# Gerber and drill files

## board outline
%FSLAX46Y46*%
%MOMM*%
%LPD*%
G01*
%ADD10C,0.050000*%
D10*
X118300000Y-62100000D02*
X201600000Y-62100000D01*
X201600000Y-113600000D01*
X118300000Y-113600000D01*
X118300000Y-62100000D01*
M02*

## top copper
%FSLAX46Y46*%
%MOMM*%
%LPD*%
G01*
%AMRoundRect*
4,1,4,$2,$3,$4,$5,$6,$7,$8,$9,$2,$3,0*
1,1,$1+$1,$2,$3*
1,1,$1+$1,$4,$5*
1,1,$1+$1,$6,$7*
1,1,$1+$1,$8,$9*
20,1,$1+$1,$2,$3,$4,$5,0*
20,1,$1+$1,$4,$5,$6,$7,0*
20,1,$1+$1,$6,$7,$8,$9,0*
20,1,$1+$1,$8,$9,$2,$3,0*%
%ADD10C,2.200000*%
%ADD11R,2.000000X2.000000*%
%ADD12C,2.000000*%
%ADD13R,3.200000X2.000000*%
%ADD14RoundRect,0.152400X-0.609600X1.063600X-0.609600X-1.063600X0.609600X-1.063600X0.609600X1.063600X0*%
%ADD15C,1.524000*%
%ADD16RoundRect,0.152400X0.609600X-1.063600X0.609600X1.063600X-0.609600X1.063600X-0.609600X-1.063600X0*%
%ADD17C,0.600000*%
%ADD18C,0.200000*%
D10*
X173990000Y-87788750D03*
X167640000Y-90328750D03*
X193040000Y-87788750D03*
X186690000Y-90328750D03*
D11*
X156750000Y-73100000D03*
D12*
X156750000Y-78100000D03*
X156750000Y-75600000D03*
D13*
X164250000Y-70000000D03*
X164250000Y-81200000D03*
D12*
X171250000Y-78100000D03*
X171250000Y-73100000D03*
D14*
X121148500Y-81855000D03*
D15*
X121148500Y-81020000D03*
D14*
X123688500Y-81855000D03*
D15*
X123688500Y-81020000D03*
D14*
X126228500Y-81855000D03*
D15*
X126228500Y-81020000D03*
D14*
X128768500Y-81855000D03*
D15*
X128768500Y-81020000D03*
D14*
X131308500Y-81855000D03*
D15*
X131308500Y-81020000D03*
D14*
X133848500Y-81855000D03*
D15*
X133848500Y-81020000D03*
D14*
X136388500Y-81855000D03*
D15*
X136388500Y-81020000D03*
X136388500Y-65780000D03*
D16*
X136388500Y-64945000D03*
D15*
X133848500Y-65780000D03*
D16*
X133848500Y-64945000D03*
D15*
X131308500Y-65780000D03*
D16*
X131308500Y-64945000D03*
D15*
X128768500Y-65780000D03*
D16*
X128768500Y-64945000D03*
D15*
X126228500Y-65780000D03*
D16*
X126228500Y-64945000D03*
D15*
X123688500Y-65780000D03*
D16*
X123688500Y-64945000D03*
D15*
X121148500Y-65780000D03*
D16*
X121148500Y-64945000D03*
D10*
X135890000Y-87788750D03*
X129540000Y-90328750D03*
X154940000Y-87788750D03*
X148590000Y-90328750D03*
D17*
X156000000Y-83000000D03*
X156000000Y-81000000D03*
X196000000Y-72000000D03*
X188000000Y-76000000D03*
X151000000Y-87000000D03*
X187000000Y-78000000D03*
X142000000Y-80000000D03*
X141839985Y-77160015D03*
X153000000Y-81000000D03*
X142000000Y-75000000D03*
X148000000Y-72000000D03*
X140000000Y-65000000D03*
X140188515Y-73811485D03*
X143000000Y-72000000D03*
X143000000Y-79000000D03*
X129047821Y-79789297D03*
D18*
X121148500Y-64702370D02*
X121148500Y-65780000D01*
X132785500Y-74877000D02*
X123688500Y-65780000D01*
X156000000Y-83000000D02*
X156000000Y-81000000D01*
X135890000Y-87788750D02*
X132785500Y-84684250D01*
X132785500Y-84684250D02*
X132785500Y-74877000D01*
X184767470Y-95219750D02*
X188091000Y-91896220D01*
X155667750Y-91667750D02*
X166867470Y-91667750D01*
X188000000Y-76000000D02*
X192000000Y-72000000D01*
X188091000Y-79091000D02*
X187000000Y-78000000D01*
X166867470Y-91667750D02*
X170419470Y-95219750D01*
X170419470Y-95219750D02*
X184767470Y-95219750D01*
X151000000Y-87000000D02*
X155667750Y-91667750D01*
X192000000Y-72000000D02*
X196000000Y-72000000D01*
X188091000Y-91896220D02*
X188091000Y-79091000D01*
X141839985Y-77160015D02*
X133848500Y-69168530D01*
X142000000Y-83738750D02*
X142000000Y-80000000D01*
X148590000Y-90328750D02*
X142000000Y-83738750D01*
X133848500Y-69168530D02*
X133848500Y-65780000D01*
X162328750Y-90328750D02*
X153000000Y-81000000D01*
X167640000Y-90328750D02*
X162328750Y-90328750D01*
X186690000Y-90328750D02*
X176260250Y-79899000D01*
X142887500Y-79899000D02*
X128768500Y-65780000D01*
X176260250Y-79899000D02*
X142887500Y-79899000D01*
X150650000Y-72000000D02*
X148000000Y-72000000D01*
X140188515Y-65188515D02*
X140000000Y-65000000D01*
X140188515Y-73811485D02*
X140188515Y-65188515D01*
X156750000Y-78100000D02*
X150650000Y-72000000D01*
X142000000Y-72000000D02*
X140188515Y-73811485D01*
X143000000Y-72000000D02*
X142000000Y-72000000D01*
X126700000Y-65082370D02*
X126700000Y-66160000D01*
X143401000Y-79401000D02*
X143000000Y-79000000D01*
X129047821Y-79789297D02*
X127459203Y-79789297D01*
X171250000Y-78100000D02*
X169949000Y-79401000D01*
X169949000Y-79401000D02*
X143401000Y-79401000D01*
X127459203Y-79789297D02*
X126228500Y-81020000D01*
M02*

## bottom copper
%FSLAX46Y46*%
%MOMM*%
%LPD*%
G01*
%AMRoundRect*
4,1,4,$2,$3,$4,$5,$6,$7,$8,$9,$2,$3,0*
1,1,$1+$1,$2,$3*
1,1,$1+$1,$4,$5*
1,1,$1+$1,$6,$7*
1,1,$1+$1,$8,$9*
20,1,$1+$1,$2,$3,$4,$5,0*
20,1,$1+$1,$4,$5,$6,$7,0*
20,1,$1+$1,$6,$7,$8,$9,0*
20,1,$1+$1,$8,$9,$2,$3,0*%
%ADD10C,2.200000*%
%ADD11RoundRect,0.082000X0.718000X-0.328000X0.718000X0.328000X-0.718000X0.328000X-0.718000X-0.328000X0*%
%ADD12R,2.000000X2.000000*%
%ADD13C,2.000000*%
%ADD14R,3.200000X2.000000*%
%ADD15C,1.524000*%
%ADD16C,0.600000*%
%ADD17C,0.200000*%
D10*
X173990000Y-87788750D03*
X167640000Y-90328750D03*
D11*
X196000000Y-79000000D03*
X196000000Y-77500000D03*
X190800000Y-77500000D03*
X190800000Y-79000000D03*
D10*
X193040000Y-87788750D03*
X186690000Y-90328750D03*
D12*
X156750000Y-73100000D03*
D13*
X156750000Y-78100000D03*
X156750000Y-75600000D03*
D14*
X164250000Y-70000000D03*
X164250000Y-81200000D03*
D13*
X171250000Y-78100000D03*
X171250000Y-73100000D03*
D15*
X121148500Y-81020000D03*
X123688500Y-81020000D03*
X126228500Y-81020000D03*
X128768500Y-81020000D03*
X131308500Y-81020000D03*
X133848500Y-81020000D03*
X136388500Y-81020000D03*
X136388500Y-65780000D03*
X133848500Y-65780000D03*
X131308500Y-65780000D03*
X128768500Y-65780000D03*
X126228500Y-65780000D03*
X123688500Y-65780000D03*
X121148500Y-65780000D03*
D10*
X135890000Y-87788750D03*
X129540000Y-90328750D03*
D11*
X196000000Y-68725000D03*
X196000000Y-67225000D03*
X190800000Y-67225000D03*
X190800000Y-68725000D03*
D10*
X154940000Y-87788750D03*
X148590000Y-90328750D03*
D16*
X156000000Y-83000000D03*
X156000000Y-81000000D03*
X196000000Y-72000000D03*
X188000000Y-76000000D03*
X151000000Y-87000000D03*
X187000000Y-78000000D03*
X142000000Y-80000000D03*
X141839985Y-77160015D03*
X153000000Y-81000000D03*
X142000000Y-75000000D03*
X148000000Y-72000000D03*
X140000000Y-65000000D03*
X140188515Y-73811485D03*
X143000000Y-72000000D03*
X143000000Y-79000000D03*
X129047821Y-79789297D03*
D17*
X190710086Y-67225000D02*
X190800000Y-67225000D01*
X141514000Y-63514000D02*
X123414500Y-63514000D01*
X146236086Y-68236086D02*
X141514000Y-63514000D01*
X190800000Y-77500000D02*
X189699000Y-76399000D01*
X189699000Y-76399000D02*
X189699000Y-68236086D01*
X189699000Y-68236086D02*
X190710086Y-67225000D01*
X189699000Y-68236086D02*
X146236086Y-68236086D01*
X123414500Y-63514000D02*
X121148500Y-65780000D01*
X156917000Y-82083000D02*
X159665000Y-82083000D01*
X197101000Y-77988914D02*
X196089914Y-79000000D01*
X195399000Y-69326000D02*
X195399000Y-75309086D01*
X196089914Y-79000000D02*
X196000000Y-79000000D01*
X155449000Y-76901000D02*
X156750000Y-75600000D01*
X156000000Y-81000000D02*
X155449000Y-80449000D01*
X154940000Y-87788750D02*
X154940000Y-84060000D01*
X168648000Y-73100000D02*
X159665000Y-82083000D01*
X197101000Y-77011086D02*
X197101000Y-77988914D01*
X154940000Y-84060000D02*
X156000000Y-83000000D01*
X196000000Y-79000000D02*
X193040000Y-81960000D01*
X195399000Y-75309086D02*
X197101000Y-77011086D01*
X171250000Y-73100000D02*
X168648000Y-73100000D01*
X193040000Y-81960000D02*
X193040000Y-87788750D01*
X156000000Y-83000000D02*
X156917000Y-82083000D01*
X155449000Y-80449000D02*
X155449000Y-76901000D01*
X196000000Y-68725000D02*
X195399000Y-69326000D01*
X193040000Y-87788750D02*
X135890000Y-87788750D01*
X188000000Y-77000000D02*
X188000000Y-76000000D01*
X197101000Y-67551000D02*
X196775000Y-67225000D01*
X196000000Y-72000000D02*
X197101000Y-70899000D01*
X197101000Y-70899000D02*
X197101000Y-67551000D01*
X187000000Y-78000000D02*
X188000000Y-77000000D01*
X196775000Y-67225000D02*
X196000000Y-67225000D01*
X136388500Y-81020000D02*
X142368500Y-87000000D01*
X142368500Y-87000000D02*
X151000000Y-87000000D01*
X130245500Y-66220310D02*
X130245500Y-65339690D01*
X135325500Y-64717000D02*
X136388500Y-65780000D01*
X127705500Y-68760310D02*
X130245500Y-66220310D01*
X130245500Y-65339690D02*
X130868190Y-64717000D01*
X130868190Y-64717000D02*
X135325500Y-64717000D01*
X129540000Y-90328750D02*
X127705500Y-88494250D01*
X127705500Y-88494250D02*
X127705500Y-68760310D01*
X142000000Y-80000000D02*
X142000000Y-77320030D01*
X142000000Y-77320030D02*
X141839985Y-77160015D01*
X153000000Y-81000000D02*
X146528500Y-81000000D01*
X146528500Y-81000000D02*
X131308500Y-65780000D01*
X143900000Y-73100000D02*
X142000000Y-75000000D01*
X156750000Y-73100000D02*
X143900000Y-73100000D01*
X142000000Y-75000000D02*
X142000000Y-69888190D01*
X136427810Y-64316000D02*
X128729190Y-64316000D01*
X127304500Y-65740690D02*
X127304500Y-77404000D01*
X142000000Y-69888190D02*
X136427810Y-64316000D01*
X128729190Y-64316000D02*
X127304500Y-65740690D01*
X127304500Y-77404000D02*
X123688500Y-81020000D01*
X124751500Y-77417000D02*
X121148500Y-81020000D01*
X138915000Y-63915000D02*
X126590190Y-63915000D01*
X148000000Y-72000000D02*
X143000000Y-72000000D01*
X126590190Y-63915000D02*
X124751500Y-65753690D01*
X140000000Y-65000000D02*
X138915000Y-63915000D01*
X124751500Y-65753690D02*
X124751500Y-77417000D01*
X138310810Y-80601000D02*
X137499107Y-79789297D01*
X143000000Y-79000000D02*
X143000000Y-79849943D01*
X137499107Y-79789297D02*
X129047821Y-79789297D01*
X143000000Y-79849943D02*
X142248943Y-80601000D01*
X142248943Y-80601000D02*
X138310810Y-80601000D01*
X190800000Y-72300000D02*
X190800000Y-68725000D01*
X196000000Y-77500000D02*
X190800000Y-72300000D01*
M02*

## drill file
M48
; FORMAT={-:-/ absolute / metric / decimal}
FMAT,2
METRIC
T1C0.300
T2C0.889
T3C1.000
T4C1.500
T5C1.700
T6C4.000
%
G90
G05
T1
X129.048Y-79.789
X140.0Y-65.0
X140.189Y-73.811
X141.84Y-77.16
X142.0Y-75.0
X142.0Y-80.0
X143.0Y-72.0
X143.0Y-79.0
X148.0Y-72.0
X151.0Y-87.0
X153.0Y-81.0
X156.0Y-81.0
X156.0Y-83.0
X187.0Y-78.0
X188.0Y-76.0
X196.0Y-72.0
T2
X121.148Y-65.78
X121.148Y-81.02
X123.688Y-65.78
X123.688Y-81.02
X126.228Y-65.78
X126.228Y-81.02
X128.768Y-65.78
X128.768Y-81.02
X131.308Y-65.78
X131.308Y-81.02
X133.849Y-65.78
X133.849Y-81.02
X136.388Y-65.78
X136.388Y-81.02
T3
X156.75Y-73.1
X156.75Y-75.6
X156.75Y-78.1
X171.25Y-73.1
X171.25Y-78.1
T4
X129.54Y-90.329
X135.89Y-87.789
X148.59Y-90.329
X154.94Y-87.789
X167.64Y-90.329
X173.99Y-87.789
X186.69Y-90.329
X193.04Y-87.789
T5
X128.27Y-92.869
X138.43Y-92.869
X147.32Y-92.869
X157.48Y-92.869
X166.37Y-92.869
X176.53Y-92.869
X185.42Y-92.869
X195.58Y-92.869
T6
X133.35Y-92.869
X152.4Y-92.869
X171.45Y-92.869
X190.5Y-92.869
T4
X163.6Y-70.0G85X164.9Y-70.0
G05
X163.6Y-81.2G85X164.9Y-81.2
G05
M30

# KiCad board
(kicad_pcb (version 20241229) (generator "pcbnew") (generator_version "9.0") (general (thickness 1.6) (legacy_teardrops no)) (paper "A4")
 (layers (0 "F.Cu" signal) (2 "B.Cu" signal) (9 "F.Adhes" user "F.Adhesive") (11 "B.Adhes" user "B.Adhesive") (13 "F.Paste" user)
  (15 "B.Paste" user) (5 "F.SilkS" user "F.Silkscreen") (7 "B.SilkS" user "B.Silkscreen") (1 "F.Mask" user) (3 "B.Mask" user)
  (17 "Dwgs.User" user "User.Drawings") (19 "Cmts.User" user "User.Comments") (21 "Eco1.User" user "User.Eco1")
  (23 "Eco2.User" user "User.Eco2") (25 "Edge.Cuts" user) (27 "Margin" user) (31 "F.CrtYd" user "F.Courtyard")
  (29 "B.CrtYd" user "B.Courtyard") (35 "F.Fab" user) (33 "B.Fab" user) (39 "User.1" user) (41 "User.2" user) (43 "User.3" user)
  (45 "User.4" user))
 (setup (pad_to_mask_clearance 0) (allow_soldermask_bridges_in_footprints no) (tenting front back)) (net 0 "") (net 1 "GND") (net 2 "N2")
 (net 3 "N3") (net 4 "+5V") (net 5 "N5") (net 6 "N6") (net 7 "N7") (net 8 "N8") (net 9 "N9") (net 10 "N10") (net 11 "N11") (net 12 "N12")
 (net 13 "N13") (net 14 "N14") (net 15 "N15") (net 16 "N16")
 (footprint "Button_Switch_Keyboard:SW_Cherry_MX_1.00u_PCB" (layer "F.Cu") (at 173.99 87.78875)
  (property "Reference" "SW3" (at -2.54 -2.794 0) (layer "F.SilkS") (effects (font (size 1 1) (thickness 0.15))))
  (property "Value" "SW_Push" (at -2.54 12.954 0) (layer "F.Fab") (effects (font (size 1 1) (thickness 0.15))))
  (pad "" np_thru_hole circle (at -7.62 5.08) (size 1.7 1.7) (drill 1.7) (layers "*.Cu" "*.Mask"))
  (pad "" np_thru_hole circle (at -2.54 5.08) (size 4 4) (drill 4) (layers "*.Cu" "*.Mask"))
  (pad "" np_thru_hole circle (at 2.54 5.08) (size 1.7 1.7) (drill 1.7) (layers "*.Cu" "*.Mask"))
  (pad "1" thru_hole circle (at 0 0) (size 2.2 2.2) (drill 1.5) (layers "*.Cu" "*.Mask") (remove_unused_layers no) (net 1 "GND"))
  (pad "2" thru_hole circle (at -6.35 2.54) (size 2.2 2.2) (drill 1.5) (layers "*.Cu" "*.Mask") (remove_unused_layers no) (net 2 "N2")))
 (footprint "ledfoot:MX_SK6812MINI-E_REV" (layer "F.Cu") (at 193.4 73.17)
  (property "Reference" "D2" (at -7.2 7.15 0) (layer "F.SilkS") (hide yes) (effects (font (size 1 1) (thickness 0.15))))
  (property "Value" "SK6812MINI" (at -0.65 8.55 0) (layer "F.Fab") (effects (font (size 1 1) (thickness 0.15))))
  (pad "1" smd roundrect (at 2.6 5.83 90) (size 0.82 1.6) (layers "B.Cu" "B.Mask" "B.Paste") (roundrect_rratio 0.1) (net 1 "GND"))
  (pad "2" smd roundrect (at 2.6 4.33 90) (size 0.82 1.6) (layers "B.Cu" "B.Mask" "B.Paste") (roundrect_rratio 0.1) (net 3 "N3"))
  (pad "3" smd roundrect (at -2.6 4.33 90) (size 0.82 1.6) (layers "B.Cu" "B.Mask" "B.Paste") (roundrect_rratio 0.1) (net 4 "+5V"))
  (pad "4" smd roundrect (at -2.6 5.83 90) (size 0.82 1.6) (layers "B.Cu" "B.Mask" "B.Paste") (roundrect_rratio 0.1) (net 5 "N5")))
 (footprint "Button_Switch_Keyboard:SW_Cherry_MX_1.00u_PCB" (layer "F.Cu") (at 193.04 87.78875)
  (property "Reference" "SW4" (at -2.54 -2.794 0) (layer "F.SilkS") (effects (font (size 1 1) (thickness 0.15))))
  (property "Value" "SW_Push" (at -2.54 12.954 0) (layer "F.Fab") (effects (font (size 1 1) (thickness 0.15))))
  (pad "" np_thru_hole circle (at -7.62 5.08) (size 1.7 1.7) (drill 1.7) (layers "*.Cu" "*.Mask"))
  (pad "" np_thru_hole circle (at -2.54 5.08) (size 4 4) (drill 4) (layers "*.Cu" "*.Mask"))
  (pad "" np_thru_hole circle (at 2.54 5.08) (size 1.7 1.7) (drill 1.7) (layers "*.Cu" "*.Mask"))
  (pad "1" thru_hole circle (at 0 0) (size 2.2 2.2) (drill 1.5) (layers "*.Cu" "*.Mask") (remove_unused_layers no) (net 1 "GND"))
  (pad "2" thru_hole circle (at -6.35 2.54) (size 2.2 2.2) (drill 1.5) (layers "*.Cu" "*.Mask") (remove_unused_layers no) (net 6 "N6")))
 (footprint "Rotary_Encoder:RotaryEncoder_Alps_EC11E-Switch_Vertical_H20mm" (layer "F.Cu") (at 156.75 73.1)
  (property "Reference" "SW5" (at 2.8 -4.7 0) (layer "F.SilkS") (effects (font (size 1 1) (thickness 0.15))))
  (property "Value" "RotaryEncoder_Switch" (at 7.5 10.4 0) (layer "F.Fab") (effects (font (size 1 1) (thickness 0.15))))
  (pad "A" thru_hole rect (at 0 0) (size 2 2) (drill 1) (layers "*.Cu" "*.Mask") (remove_unused_layers no) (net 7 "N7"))
  (pad "B" thru_hole circle (at 0 5) (size 2 2) (drill 1) (layers "*.Cu" "*.Mask") (remove_unused_layers no) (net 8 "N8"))
  (pad "C" thru_hole circle (at 0 2.5) (size 2 2) (drill 1) (layers "*.Cu" "*.Mask") (remove_unused_layers no) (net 1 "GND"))
  (pad "MP" thru_hole rect (at 7.5 -3.1) (size 3.2 2) (drill oval 2.8 1.5) (layers "*.Cu" "*.Mask") (remove_unused_layers no))
  (pad "MP" thru_hole rect (at 7.5 8.1) (size 3.2 2) (drill oval 2.8 1.5) (layers "*.Cu" "*.Mask") (remove_unused_layers no))
  (pad "S1" thru_hole circle (at 14.5 5) (size 2 2) (drill 1) (layers "*.Cu" "*.Mask") (remove_unused_layers no) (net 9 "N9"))
  (pad "S2" thru_hole circle (at 14.5 0) (size 2 2) (drill 1) (layers "*.Cu" "*.Mask") (remove_unused_layers no) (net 1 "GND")))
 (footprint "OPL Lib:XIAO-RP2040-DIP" (layer "F.Cu") (at 128.7685 73.4 90)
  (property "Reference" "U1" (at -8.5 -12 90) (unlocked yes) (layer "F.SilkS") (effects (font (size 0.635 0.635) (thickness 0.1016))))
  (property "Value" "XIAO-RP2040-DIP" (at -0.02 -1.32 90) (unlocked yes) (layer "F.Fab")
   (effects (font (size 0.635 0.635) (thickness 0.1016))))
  (pad "1" smd roundrect (at -8.455 -7.62 270) (size 2.432 1.524) (layers "F.Cu" "F.Mask") (roundrect_rratio 0.1) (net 8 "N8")
   (thermal_bridge_angle 45))
  (pad "1" thru_hole circle (at -7.62 -7.62 270) (size 1.524 1.524) (drill 0.889) (layers "*.Cu" "*.Mask") (remove_unused_layers no)
   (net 8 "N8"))
  (pad "2" smd roundrect (at -8.455 -5.08 270) (size 2.432 1.524) (layers "F.Cu" "F.Mask") (roundrect_rratio 0.1) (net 7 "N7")
   (thermal_bridge_angle 45))
  (pad "2" thru_hole circle (at -7.62 -5.08 270) (size 1.524 1.524) (drill 0.889) (layers "*.Cu" "*.Mask") (remove_unused_layers no)
   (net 7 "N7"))
  (pad "3" smd roundrect (at -8.455 -2.54 270) (size 2.432 1.524) (layers "F.Cu" "F.Mask") (roundrect_rratio 0.1) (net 9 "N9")
   (thermal_bridge_angle 45))
  (pad "3" thru_hole circle (at -7.62 -2.54 270) (size 1.524 1.524) (drill 0.889) (layers "*.Cu" "*.Mask") (remove_unused_layers no)
   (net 9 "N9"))
  (pad "4" smd roundrect (at -8.455 0 270) (size 2.432 1.524) (layers "F.Cu" "F.Mask") (roundrect_rratio 0.1) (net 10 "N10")
   (thermal_bridge_angle 45))
  (pad "4" thru_hole circle (at -7.62 0 270) (size 1.524 1.524) (drill 0.889) (layers "*.Cu" "*.Mask") (remove_unused_layers no)
   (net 10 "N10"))
  (pad "5" smd roundrect (at -8.455 2.54 270) (size 2.432 1.524) (layers "F.Cu" "F.Mask") (roundrect_rratio 0.1) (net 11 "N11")
   (thermal_bridge_angle 45))
  (pad "5" thru_hole circle (at -7.62 2.54 270) (size 1.524 1.524) (drill 0.889) (layers "*.Cu" "*.Mask") (remove_unused_layers no)
   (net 11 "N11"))
  (pad "6" smd roundrect (at -8.455 5.08 270) (size 2.432 1.524) (layers "F.Cu" "F.Mask") (roundrect_rratio 0.1) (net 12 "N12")
   (thermal_bridge_angle 45))
  (pad "6" thru_hole circle (at -7.62 5.08 270) (size 1.524 1.524) (drill 0.889) (layers "*.Cu" "*.Mask") (remove_unused_layers no)
   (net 12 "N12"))
  (pad "7" smd roundrect (at -8.455 7.62 270) (size 2.432 1.524) (layers "F.Cu" "F.Mask") (roundrect_rratio 0.1) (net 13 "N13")
   (thermal_bridge_angle 45))
  (pad "7" thru_hole circle (at -7.62 7.62 270) (size 1.524 1.524) (drill 0.889) (layers "*.Cu" "*.Mask") (remove_unused_layers no)
   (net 13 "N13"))
  (pad "8" thru_hole circle (at 7.62 7.62 90) (size 1.524 1.524) (drill 0.889) (layers "*.Cu" "*.Mask") (remove_unused_layers no)
   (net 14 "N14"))
  (pad "8" smd roundrect (at 8.455 7.62 90) (size 2.432 1.524) (layers "F.Cu" "F.Mask") (roundrect_rratio 0.1) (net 14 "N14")
   (thermal_bridge_angle 45))
  (pad "9" thru_hole circle (at 7.62 5.08 90) (size 1.524 1.524) (drill 0.889) (layers "*.Cu" "*.Mask") (remove_unused_layers no)
   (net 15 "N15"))
  (pad "9" smd roundrect (at 8.455 5.08 90) (size 2.432 1.524) (layers "F.Cu" "F.Mask") (roundrect_rratio 0.1) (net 15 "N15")
   (thermal_bridge_angle 45))
  (pad "10" thru_hole circle (at 7.62 2.54 90) (size 1.524 1.524) (drill 0.889) (layers "*.Cu" "*.Mask") (remove_unused_layers no)
   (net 2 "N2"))
  (pad "10" smd roundrect (at 8.455 2.54 90) (size 2.432 1.524) (layers "F.Cu" "F.Mask") (roundrect_rratio 0.1) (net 2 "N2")
   (thermal_bridge_angle 45))
  (pad "11" thru_hole circle (at 7.62 0 90) (size 1.524 1.524) (drill 0.889) (layers "*.Cu" "*.Mask") (remove_unused_layers no) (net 6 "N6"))
  (pad "11" smd roundrect (at 8.455 0 90) (size 2.432 1.524) (layers "F.Cu" "F.Mask") (roundrect_rratio 0.1) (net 6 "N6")
   (thermal_bridge_angle 45))
  (pad "12" thru_hole circle (at 7.62 -2.54 90) (size 1.524 1.524) (drill 0.889) (layers "*.Cu" "*.Mask") (remove_unused_layers no)
   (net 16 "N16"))
  (pad "12" smd roundrect (at 8.455 -2.54 90) (size 2.432 1.524) (layers "F.Cu" "F.Mask") (roundrect_rratio 0.1) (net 16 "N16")
   (thermal_bridge_angle 45))
  (pad "13" thru_hole circle (at 7.62 -5.08 90) (size 1.524 1.524) (drill 0.889) (layers "*.Cu" "*.Mask") (remove_unused_layers no)
   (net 1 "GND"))
  (pad "13" smd roundrect (at 8.455 -5.08 90) (size 2.432 1.524) (layers "F.Cu" "F.Mask") (roundrect_rratio 0.1) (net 1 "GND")
   (thermal_bridge_angle 45))
  (pad "14" thru_hole circle (at 7.62 -7.62 90) (size 1.524 1.524) (drill 0.889) (layers "*.Cu" "*.Mask") (remove_unused_layers no)
   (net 4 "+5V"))
  (pad "14" smd roundrect (at 8.455 -7.62 90) (size 2.432 1.524) (layers "F.Cu" "F.Mask") (roundrect_rratio 0.1) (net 4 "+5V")
   (thermal_bridge_angle 45)))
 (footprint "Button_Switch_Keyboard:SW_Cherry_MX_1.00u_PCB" (layer "F.Cu") (at 135.89 87.78875)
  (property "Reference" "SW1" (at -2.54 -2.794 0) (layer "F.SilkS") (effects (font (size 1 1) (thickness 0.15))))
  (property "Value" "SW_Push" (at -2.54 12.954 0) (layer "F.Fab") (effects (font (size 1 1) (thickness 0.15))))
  (pad "" np_thru_hole circle (at -7.62 5.08) (size 1.7 1.7) (drill 1.7) (layers "*.Cu" "*.Mask"))
  (pad "" np_thru_hole circle (at -2.54 5.08) (size 4 4) (drill 4) (layers "*.Cu" "*.Mask"))
  (pad "" np_thru_hole circle (at 2.54 5.08) (size 1.7 1.7) (drill 1.7) (layers "*.Cu" "*.Mask"))
  (pad "1" thru_hole circle (at 0 0) (size 2.2 2.2) (drill 1.5) (layers "*.Cu" "*.Mask") (remove_unused_layers no) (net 1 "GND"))
  (pad "2" thru_hole circle (at -6.35 2.54) (size 2.2 2.2) (drill 1.5) (layers "*.Cu" "*.Mask") (remove_unused_layers no) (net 14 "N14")))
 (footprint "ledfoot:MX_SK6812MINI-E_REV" (layer "F.Cu") (at 193.4 62.895)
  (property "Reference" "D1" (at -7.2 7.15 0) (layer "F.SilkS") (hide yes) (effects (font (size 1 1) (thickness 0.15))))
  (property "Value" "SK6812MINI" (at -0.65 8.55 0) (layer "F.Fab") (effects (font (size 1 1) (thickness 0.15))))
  (pad "1" smd roundrect (at 2.6 5.83 90) (size 0.82 1.6) (layers "B.Cu" "B.Mask" "B.Paste") (roundrect_rratio 0.1) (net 1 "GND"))
  (pad "2" smd roundrect (at 2.6 4.33 90) (size 0.82 1.6) (layers "B.Cu" "B.Mask" "B.Paste") (roundrect_rratio 0.1) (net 13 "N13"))
  (pad "3" smd roundrect (at -2.6 4.33 90) (size 0.82 1.6) (layers "B.Cu" "B.Mask" "B.Paste") (roundrect_rratio 0.1) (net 4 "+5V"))
  (pad "4" smd roundrect (at -2.6 5.83 90) (size 0.82 1.6) (layers "B.Cu" "B.Mask" "B.Paste") (roundrect_rratio 0.1) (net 3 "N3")))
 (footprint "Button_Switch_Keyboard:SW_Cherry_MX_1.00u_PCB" (layer "F.Cu") (at 154.94 87.78875)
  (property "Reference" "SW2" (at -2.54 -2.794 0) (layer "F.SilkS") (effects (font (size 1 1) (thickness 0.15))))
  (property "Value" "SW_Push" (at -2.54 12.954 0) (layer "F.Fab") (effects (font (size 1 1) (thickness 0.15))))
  (pad "" np_thru_hole circle (at -7.62 5.08) (size 1.7 1.7) (drill 1.7) (layers "*.Cu" "*.Mask"))
  (pad "" np_thru_hole circle (at -2.54 5.08) (size 4 4) (drill 4) (layers "*.Cu" "*.Mask"))
  (pad "" np_thru_hole circle (at 2.54 5.08) (size 1.7 1.7) (drill 1.7) (layers "*.Cu" "*.Mask"))
  (pad "1" thru_hole circle (at 0 0) (size 2.2 2.2) (drill 1.5) (layers "*.Cu" "*.Mask") (remove_unused_layers no) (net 1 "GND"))
  (pad "2" thru_hole circle (at -6.35 2.54) (size 2.2 2.2) (drill 1.5) (layers "*.Cu" "*.Mask") (remove_unused_layers no) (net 15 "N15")))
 (gr_rect (start 118.3 62.1) (end 201.6 113.6) (stroke (width 0.05) (type default)) (fill no) (layer "Edge.Cuts"))
 (segment (start 121.1485 64.70237) (end 121.1485 65.78) (width 0.2) (layer "F.Cu") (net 4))
 (segment (start 190.710086 67.225) (end 190.8 67.225) (width 0.2) (layer "B.Cu") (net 4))
 (segment (start 141.514 63.514) (end 123.4145 63.514) (width 0.2) (layer "B.Cu") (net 4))
 (segment (start 146.236086 68.236086) (end 141.514 63.514) (width 0.2) (layer "B.Cu") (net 4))
 (segment (start 190.8 77.5) (end 189.699 76.399) (width 0.2) (layer "B.Cu") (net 4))
 (segment (start 189.699 76.399) (end 189.699 68.236086) (width 0.2) (layer "B.Cu") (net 4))
 (segment (start 189.699 68.236086) (end 190.710086 67.225) (width 0.2) (layer "B.Cu") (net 4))
 (segment (start 189.699 68.236086) (end 146.236086 68.236086) (width 0.2) (layer "B.Cu") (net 4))
 (segment (start 123.4145 63.514) (end 121.1485 65.78) (width 0.2) (layer "B.Cu") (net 4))
 (segment (start 132.7855 74.877) (end 123.6885 65.78) (width 0.2) (layer "F.Cu") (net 1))
 (segment (start 156 83) (end 156 81) (width 0.2) (layer "F.Cu") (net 1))
 (segment (start 135.89 87.78875) (end 132.7855 84.68425) (width 0.2) (layer "F.Cu") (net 1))
 (segment (start 132.7855 84.68425) (end 132.7855 74.877) (width 0.2) (layer "F.Cu") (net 1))
 (via (at 156 83) (size 0.6) (drill 0.3) (layers "F.Cu" "B.Cu") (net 1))
 (via (at 156 81) (size 0.6) (drill 0.3) (layers "F.Cu" "B.Cu") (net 1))
 (segment (start 156.917 82.083) (end 159.665 82.083) (width 0.2) (layer "B.Cu") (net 1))
 (segment (start 197.101 77.988914) (end 196.089914 79) (width 0.2) (layer "B.Cu") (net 1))
 (segment (start 195.399 69.326) (end 195.399 75.309086) (width 0.2) (layer "B.Cu") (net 1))
 (segment (start 196.089914 79) (end 196 79) (width 0.2) (layer "B.Cu") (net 1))
 (segment (start 155.449 76.901) (end 156.75 75.6) (width 0.2) (layer "B.Cu") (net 1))
 (segment (start 156 81) (end 155.449 80.449) (width 0.2) (layer "B.Cu") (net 1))
 (segment (start 154.94 87.78875) (end 154.94 84.06) (width 0.2) (layer "B.Cu") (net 1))
 (segment (start 168.648 73.1) (end 159.665 82.083) (width 0.2) (layer "B.Cu") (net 1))
 (segment (start 197.101 77.011086) (end 197.101 77.988914) (width 0.2) (layer "B.Cu") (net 1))
 (segment (start 154.94 84.06) (end 156 83) (width 0.2) (layer "B.Cu") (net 1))
 (segment (start 196 79) (end 193.04 81.96) (width 0.2) (layer "B.Cu") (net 1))
 (segment (start 195.399 75.309086) (end 197.101 77.011086) (width 0.2) (layer "B.Cu") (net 1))
 (segment (start 171.25 73.1) (end 168.648 73.1) (width 0.2) (layer "B.Cu") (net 1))
 (segment (start 193.04 81.96) (end 193.04 87.78875) (width 0.2) (layer "B.Cu") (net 1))
 (segment (start 156 83) (end 156.917 82.083) (width 0.2) (layer "B.Cu") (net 1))
 (segment (start 155.449 80.449) (end 155.449 76.901) (width 0.2) (layer "B.Cu") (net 1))
 (segment (start 196 68.725) (end 195.399 69.326) (width 0.2) (layer "B.Cu") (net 1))
 (segment (start 193.04 87.78875) (end 135.89 87.78875) (width 0.2) (layer "B.Cu") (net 1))
 (segment (start 184.76747 95.21975) (end 188.091 91.89622) (width 0.2) (layer "F.Cu") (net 13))
 (segment (start 155.66775 91.66775) (end 166.86747 91.66775) (width 0.2) (layer "F.Cu") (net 13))
 (segment (start 188 76) (end 192 72) (width 0.2) (layer "F.Cu") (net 13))
 (segment (start 188.091 79.091) (end 187 78) (width 0.2) (layer "F.Cu") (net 13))
 (segment (start 166.86747 91.66775) (end 170.41947 95.21975) (width 0.2) (layer "F.Cu") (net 13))
 (segment (start 170.41947 95.21975) (end 184.76747 95.21975) (width 0.2) (layer "F.Cu") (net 13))
 (segment (start 151 87) (end 155.66775 91.66775) (width 0.2) (layer "F.Cu") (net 13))
 (segment (start 192 72) (end 196 72) (width 0.2) (layer "F.Cu") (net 13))
 (segment (start 188.091 91.89622) (end 188.091 79.091) (width 0.2) (layer "F.Cu") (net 13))
 (via (at 196 72) (size 0.6) (drill 0.3) (layers "F.Cu" "B.Cu") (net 13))
 (via (at 188 76) (size 0.6) (drill 0.3) (layers "F.Cu" "B.Cu") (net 13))
 (via (at 151 87) (size 0.6) (drill 0.3) (layers "F.Cu" "B.Cu") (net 13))
 (via (at 187 78) (size 0.6) (drill 0.3) (layers "F.Cu" "B.Cu") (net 13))
 (segment (start 188 77) (end 188 76) (width 0.2) (layer "B.Cu") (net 13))
 (segment (start 197.101 67.551) (end 196.775 67.225) (width 0.2) (layer "B.Cu") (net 13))
 (segment (start 196 72) (end 197.101 70.899) (width 0.2) (layer "B.Cu") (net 13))
 (segment (start 197.101 70.899) (end 197.101 67.551) (width 0.2) (layer "B.Cu") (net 13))
 (segment (start 187 78) (end 188 77) (width 0.2) (layer "B.Cu") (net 13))
 (segment (start 196.775 67.225) (end 196 67.225) (width 0.2) (layer "B.Cu") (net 13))
 (segment (start 136.3885 81.02) (end 142.3685 87) (width 0.2) (layer "B.Cu") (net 13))
 (segment (start 142.3685 87) (end 151 87) (width 0.2) (layer "B.Cu") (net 13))
 (segment (start 130.2455 66.22031) (end 130.2455 65.33969) (width 0.2) (layer "B.Cu") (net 14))
 (segment (start 135.3255 64.717) (end 136.3885 65.78) (width 0.2) (layer "B.Cu") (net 14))
 (segment (start 127.7055 68.76031) (end 130.2455 66.22031) (width 0.2) (layer "B.Cu") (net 14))
 (segment (start 130.2455 65.33969) (end 130.86819 64.717) (width 0.2) (layer "B.Cu") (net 14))
 (segment (start 130.86819 64.717) (end 135.3255 64.717) (width 0.2) (layer "B.Cu") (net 14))
 (segment (start 129.54 90.32875) (end 127.7055 88.49425) (width 0.2) (layer "B.Cu") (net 14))
 (segment (start 127.7055 88.49425) (end 127.7055 68.76031) (width 0.2) (layer "B.Cu") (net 14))
 (segment (start 141.839985 77.160015) (end 133.8485 69.16853) (width 0.2) (layer "F.Cu") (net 15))
 (segment (start 142 83.73875) (end 142 80) (width 0.2) (layer "F.Cu") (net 15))
 (segment (start 148.59 90.32875) (end 142 83.73875) (width 0.2) (layer "F.Cu") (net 15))
 (segment (start 133.8485 69.16853) (end 133.8485 65.78) (width 0.2) (layer "F.Cu") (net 15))
 (via (at 142 80) (size 0.6) (drill 0.3) (layers "F.Cu" "B.Cu") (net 15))
 (via (at 141.839985 77.160015) (size 0.6) (drill 0.3) (layers "F.Cu" "B.Cu") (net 15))
 (segment (start 142 80) (end 142 77.32003) (width 0.2) (layer "B.Cu") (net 15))
 (segment (start 142 77.32003) (end 141.839985 77.160015) (width 0.2) (layer "B.Cu") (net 15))
 (segment (start 162.32875 90.32875) (end 153 81) (width 0.2) (layer "F.Cu") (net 2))
 (segment (start 167.64 90.32875) (end 162.32875 90.32875) (width 0.2) (layer "F.Cu") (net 2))
 (via (at 153 81) (size 0.6) (drill 0.3) (layers "F.Cu" "B.Cu") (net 2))
 (segment (start 153 81) (end 146.5285 81) (width 0.2) (layer "B.Cu") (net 2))
 (segment (start 146.5285 81) (end 131.3085 65.78) (width 0.2) (layer "B.Cu") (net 2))
 (segment (start 186.69 90.32875) (end 176.26025 79.899) (width 0.2) (layer "F.Cu") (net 6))
 (segment (start 142.8875 79.899) (end 128.7685 65.78) (width 0.2) (layer "F.Cu") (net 6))
 (segment (start 176.26025 79.899) (end 142.8875 79.899) (width 0.2) (layer "F.Cu") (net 6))
 (via (at 142 75) (size 0.6) (drill 0.3) (layers "F.Cu" "B.Cu") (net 7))
 (segment (start 143.9 73.1) (end 142 75) (width 0.2) (layer "B.Cu") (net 7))
 (segment (start 156.75 73.1) (end 143.9 73.1) (width 0.2) (layer "B.Cu") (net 7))
 (segment (start 142 75) (end 142 69.88819) (width 0.2) (layer "B.Cu") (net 7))
 (segment (start 136.42781 64.316) (end 128.72919 64.316) (width 0.2) (layer "B.Cu") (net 7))
 (segment (start 127.3045 65.74069) (end 127.3045 77.404) (width 0.2) (layer "B.Cu") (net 7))
 (segment (start 142 69.88819) (end 136.42781 64.316) (width 0.2) (layer "B.Cu") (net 7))
 (segment (start 128.72919 64.316) (end 127.3045 65.74069) (width 0.2) (layer "B.Cu") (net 7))
 (segment (start 127.3045 77.404) (end 123.6885 81.02) (width 0.2) (layer "B.Cu") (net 7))
 (segment (start 150.65 72) (end 148 72) (width 0.2) (layer "F.Cu") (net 8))
 (segment (start 140.188515 65.188515) (end 140 65) (width 0.2) (layer "F.Cu") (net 8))
 (segment (start 140.188515 73.811485) (end 140.188515 65.188515) (width 0.2) (layer "F.Cu") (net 8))
 (segment (start 156.75 78.1) (end 150.65 72) (width 0.2) (layer "F.Cu") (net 8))
 (segment (start 142 72) (end 140.188515 73.811485) (width 0.2) (layer "F.Cu") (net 8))
 (segment (start 143 72) (end 142 72) (width 0.2) (layer "F.Cu") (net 8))
 (via (at 148 72) (size 0.6) (drill 0.3) (layers "F.Cu" "B.Cu") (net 8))
 (via (at 140 65) (size 0.6) (drill 0.3) (layers "F.Cu" "B.Cu") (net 8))
 (via (at 140.188515 73.811485) (size 0.6) (drill 0.3) (layers "F.Cu" "B.Cu") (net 8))
 (via (at 143 72) (size 0.6) (drill 0.3) (layers "F.Cu" "B.Cu") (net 8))
 (segment (start 124.7515 77.417) (end 121.1485 81.02) (width 0.2) (layer "B.Cu") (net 8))
 (segment (start 138.915 63.915) (end 126.59019 63.915) (width 0.2) (layer "B.Cu") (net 8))
 (segment (start 148 72) (end 143 72) (width 0.2) (layer "B.Cu") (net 8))
 (segment (start 126.59019 63.915) (end 124.7515 65.75369) (width 0.2) (layer "B.Cu") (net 8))
 (segment (start 140 65) (end 138.915 63.915) (width 0.2) (layer "B.Cu") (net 8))
 (segment (start 124.7515 65.75369) (end 124.7515 77.417) (width 0.2) (layer "B.Cu") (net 8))
 (segment (start 126.7 65.08237) (end 126.7 66.16) (width 0.2) (layer "F.Cu") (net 16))
 (segment (start 143.401 79.401) (end 143 79) (width 0.2) (layer "F.Cu") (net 9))
 (segment (start 129.047821 79.789297) (end 127.459203 79.789297) (width 0.2) (layer "F.Cu") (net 9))
 (segment (start 171.25 78.1) (end 169.949 79.401) (width 0.2) (layer "F.Cu") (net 9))
 (segment (start 169.949 79.401) (end 143.401 79.401) (width 0.2) (layer "F.Cu") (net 9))
 (segment (start 127.459203 79.789297) (end 126.2285 81.02) (width 0.2) (layer "F.Cu") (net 9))
 (via (at 143 79) (size 0.6) (drill 0.3) (layers "F.Cu" "B.Cu") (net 9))
 (via (at 129.047821 79.789297) (size 0.6) (drill 0.3) (layers "F.Cu" "B.Cu") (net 9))
 (segment (start 138.31081 80.601) (end 137.499107 79.789297) (width 0.2) (layer "B.Cu") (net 9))
 (segment (start 143 79) (end 143 79.849943) (width 0.2) (layer "B.Cu") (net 9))
 (segment (start 137.499107 79.789297) (end 129.047821 79.789297) (width 0.2) (layer "B.Cu") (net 9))
 (segment (start 143 79.849943) (end 142.248943 80.601) (width 0.2) (layer "B.Cu") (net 9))
 (segment (start 142.248943 80.601) (end 138.31081 80.601) (width 0.2) (layer "B.Cu") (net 9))
 (segment (start 190.8 72.3) (end 190.8 68.725) (width 0.2) (layer "B.Cu") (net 3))
 (segment (start 196 77.5) (end 190.8 72.3) (width 0.2) (layer "B.Cu") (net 3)))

